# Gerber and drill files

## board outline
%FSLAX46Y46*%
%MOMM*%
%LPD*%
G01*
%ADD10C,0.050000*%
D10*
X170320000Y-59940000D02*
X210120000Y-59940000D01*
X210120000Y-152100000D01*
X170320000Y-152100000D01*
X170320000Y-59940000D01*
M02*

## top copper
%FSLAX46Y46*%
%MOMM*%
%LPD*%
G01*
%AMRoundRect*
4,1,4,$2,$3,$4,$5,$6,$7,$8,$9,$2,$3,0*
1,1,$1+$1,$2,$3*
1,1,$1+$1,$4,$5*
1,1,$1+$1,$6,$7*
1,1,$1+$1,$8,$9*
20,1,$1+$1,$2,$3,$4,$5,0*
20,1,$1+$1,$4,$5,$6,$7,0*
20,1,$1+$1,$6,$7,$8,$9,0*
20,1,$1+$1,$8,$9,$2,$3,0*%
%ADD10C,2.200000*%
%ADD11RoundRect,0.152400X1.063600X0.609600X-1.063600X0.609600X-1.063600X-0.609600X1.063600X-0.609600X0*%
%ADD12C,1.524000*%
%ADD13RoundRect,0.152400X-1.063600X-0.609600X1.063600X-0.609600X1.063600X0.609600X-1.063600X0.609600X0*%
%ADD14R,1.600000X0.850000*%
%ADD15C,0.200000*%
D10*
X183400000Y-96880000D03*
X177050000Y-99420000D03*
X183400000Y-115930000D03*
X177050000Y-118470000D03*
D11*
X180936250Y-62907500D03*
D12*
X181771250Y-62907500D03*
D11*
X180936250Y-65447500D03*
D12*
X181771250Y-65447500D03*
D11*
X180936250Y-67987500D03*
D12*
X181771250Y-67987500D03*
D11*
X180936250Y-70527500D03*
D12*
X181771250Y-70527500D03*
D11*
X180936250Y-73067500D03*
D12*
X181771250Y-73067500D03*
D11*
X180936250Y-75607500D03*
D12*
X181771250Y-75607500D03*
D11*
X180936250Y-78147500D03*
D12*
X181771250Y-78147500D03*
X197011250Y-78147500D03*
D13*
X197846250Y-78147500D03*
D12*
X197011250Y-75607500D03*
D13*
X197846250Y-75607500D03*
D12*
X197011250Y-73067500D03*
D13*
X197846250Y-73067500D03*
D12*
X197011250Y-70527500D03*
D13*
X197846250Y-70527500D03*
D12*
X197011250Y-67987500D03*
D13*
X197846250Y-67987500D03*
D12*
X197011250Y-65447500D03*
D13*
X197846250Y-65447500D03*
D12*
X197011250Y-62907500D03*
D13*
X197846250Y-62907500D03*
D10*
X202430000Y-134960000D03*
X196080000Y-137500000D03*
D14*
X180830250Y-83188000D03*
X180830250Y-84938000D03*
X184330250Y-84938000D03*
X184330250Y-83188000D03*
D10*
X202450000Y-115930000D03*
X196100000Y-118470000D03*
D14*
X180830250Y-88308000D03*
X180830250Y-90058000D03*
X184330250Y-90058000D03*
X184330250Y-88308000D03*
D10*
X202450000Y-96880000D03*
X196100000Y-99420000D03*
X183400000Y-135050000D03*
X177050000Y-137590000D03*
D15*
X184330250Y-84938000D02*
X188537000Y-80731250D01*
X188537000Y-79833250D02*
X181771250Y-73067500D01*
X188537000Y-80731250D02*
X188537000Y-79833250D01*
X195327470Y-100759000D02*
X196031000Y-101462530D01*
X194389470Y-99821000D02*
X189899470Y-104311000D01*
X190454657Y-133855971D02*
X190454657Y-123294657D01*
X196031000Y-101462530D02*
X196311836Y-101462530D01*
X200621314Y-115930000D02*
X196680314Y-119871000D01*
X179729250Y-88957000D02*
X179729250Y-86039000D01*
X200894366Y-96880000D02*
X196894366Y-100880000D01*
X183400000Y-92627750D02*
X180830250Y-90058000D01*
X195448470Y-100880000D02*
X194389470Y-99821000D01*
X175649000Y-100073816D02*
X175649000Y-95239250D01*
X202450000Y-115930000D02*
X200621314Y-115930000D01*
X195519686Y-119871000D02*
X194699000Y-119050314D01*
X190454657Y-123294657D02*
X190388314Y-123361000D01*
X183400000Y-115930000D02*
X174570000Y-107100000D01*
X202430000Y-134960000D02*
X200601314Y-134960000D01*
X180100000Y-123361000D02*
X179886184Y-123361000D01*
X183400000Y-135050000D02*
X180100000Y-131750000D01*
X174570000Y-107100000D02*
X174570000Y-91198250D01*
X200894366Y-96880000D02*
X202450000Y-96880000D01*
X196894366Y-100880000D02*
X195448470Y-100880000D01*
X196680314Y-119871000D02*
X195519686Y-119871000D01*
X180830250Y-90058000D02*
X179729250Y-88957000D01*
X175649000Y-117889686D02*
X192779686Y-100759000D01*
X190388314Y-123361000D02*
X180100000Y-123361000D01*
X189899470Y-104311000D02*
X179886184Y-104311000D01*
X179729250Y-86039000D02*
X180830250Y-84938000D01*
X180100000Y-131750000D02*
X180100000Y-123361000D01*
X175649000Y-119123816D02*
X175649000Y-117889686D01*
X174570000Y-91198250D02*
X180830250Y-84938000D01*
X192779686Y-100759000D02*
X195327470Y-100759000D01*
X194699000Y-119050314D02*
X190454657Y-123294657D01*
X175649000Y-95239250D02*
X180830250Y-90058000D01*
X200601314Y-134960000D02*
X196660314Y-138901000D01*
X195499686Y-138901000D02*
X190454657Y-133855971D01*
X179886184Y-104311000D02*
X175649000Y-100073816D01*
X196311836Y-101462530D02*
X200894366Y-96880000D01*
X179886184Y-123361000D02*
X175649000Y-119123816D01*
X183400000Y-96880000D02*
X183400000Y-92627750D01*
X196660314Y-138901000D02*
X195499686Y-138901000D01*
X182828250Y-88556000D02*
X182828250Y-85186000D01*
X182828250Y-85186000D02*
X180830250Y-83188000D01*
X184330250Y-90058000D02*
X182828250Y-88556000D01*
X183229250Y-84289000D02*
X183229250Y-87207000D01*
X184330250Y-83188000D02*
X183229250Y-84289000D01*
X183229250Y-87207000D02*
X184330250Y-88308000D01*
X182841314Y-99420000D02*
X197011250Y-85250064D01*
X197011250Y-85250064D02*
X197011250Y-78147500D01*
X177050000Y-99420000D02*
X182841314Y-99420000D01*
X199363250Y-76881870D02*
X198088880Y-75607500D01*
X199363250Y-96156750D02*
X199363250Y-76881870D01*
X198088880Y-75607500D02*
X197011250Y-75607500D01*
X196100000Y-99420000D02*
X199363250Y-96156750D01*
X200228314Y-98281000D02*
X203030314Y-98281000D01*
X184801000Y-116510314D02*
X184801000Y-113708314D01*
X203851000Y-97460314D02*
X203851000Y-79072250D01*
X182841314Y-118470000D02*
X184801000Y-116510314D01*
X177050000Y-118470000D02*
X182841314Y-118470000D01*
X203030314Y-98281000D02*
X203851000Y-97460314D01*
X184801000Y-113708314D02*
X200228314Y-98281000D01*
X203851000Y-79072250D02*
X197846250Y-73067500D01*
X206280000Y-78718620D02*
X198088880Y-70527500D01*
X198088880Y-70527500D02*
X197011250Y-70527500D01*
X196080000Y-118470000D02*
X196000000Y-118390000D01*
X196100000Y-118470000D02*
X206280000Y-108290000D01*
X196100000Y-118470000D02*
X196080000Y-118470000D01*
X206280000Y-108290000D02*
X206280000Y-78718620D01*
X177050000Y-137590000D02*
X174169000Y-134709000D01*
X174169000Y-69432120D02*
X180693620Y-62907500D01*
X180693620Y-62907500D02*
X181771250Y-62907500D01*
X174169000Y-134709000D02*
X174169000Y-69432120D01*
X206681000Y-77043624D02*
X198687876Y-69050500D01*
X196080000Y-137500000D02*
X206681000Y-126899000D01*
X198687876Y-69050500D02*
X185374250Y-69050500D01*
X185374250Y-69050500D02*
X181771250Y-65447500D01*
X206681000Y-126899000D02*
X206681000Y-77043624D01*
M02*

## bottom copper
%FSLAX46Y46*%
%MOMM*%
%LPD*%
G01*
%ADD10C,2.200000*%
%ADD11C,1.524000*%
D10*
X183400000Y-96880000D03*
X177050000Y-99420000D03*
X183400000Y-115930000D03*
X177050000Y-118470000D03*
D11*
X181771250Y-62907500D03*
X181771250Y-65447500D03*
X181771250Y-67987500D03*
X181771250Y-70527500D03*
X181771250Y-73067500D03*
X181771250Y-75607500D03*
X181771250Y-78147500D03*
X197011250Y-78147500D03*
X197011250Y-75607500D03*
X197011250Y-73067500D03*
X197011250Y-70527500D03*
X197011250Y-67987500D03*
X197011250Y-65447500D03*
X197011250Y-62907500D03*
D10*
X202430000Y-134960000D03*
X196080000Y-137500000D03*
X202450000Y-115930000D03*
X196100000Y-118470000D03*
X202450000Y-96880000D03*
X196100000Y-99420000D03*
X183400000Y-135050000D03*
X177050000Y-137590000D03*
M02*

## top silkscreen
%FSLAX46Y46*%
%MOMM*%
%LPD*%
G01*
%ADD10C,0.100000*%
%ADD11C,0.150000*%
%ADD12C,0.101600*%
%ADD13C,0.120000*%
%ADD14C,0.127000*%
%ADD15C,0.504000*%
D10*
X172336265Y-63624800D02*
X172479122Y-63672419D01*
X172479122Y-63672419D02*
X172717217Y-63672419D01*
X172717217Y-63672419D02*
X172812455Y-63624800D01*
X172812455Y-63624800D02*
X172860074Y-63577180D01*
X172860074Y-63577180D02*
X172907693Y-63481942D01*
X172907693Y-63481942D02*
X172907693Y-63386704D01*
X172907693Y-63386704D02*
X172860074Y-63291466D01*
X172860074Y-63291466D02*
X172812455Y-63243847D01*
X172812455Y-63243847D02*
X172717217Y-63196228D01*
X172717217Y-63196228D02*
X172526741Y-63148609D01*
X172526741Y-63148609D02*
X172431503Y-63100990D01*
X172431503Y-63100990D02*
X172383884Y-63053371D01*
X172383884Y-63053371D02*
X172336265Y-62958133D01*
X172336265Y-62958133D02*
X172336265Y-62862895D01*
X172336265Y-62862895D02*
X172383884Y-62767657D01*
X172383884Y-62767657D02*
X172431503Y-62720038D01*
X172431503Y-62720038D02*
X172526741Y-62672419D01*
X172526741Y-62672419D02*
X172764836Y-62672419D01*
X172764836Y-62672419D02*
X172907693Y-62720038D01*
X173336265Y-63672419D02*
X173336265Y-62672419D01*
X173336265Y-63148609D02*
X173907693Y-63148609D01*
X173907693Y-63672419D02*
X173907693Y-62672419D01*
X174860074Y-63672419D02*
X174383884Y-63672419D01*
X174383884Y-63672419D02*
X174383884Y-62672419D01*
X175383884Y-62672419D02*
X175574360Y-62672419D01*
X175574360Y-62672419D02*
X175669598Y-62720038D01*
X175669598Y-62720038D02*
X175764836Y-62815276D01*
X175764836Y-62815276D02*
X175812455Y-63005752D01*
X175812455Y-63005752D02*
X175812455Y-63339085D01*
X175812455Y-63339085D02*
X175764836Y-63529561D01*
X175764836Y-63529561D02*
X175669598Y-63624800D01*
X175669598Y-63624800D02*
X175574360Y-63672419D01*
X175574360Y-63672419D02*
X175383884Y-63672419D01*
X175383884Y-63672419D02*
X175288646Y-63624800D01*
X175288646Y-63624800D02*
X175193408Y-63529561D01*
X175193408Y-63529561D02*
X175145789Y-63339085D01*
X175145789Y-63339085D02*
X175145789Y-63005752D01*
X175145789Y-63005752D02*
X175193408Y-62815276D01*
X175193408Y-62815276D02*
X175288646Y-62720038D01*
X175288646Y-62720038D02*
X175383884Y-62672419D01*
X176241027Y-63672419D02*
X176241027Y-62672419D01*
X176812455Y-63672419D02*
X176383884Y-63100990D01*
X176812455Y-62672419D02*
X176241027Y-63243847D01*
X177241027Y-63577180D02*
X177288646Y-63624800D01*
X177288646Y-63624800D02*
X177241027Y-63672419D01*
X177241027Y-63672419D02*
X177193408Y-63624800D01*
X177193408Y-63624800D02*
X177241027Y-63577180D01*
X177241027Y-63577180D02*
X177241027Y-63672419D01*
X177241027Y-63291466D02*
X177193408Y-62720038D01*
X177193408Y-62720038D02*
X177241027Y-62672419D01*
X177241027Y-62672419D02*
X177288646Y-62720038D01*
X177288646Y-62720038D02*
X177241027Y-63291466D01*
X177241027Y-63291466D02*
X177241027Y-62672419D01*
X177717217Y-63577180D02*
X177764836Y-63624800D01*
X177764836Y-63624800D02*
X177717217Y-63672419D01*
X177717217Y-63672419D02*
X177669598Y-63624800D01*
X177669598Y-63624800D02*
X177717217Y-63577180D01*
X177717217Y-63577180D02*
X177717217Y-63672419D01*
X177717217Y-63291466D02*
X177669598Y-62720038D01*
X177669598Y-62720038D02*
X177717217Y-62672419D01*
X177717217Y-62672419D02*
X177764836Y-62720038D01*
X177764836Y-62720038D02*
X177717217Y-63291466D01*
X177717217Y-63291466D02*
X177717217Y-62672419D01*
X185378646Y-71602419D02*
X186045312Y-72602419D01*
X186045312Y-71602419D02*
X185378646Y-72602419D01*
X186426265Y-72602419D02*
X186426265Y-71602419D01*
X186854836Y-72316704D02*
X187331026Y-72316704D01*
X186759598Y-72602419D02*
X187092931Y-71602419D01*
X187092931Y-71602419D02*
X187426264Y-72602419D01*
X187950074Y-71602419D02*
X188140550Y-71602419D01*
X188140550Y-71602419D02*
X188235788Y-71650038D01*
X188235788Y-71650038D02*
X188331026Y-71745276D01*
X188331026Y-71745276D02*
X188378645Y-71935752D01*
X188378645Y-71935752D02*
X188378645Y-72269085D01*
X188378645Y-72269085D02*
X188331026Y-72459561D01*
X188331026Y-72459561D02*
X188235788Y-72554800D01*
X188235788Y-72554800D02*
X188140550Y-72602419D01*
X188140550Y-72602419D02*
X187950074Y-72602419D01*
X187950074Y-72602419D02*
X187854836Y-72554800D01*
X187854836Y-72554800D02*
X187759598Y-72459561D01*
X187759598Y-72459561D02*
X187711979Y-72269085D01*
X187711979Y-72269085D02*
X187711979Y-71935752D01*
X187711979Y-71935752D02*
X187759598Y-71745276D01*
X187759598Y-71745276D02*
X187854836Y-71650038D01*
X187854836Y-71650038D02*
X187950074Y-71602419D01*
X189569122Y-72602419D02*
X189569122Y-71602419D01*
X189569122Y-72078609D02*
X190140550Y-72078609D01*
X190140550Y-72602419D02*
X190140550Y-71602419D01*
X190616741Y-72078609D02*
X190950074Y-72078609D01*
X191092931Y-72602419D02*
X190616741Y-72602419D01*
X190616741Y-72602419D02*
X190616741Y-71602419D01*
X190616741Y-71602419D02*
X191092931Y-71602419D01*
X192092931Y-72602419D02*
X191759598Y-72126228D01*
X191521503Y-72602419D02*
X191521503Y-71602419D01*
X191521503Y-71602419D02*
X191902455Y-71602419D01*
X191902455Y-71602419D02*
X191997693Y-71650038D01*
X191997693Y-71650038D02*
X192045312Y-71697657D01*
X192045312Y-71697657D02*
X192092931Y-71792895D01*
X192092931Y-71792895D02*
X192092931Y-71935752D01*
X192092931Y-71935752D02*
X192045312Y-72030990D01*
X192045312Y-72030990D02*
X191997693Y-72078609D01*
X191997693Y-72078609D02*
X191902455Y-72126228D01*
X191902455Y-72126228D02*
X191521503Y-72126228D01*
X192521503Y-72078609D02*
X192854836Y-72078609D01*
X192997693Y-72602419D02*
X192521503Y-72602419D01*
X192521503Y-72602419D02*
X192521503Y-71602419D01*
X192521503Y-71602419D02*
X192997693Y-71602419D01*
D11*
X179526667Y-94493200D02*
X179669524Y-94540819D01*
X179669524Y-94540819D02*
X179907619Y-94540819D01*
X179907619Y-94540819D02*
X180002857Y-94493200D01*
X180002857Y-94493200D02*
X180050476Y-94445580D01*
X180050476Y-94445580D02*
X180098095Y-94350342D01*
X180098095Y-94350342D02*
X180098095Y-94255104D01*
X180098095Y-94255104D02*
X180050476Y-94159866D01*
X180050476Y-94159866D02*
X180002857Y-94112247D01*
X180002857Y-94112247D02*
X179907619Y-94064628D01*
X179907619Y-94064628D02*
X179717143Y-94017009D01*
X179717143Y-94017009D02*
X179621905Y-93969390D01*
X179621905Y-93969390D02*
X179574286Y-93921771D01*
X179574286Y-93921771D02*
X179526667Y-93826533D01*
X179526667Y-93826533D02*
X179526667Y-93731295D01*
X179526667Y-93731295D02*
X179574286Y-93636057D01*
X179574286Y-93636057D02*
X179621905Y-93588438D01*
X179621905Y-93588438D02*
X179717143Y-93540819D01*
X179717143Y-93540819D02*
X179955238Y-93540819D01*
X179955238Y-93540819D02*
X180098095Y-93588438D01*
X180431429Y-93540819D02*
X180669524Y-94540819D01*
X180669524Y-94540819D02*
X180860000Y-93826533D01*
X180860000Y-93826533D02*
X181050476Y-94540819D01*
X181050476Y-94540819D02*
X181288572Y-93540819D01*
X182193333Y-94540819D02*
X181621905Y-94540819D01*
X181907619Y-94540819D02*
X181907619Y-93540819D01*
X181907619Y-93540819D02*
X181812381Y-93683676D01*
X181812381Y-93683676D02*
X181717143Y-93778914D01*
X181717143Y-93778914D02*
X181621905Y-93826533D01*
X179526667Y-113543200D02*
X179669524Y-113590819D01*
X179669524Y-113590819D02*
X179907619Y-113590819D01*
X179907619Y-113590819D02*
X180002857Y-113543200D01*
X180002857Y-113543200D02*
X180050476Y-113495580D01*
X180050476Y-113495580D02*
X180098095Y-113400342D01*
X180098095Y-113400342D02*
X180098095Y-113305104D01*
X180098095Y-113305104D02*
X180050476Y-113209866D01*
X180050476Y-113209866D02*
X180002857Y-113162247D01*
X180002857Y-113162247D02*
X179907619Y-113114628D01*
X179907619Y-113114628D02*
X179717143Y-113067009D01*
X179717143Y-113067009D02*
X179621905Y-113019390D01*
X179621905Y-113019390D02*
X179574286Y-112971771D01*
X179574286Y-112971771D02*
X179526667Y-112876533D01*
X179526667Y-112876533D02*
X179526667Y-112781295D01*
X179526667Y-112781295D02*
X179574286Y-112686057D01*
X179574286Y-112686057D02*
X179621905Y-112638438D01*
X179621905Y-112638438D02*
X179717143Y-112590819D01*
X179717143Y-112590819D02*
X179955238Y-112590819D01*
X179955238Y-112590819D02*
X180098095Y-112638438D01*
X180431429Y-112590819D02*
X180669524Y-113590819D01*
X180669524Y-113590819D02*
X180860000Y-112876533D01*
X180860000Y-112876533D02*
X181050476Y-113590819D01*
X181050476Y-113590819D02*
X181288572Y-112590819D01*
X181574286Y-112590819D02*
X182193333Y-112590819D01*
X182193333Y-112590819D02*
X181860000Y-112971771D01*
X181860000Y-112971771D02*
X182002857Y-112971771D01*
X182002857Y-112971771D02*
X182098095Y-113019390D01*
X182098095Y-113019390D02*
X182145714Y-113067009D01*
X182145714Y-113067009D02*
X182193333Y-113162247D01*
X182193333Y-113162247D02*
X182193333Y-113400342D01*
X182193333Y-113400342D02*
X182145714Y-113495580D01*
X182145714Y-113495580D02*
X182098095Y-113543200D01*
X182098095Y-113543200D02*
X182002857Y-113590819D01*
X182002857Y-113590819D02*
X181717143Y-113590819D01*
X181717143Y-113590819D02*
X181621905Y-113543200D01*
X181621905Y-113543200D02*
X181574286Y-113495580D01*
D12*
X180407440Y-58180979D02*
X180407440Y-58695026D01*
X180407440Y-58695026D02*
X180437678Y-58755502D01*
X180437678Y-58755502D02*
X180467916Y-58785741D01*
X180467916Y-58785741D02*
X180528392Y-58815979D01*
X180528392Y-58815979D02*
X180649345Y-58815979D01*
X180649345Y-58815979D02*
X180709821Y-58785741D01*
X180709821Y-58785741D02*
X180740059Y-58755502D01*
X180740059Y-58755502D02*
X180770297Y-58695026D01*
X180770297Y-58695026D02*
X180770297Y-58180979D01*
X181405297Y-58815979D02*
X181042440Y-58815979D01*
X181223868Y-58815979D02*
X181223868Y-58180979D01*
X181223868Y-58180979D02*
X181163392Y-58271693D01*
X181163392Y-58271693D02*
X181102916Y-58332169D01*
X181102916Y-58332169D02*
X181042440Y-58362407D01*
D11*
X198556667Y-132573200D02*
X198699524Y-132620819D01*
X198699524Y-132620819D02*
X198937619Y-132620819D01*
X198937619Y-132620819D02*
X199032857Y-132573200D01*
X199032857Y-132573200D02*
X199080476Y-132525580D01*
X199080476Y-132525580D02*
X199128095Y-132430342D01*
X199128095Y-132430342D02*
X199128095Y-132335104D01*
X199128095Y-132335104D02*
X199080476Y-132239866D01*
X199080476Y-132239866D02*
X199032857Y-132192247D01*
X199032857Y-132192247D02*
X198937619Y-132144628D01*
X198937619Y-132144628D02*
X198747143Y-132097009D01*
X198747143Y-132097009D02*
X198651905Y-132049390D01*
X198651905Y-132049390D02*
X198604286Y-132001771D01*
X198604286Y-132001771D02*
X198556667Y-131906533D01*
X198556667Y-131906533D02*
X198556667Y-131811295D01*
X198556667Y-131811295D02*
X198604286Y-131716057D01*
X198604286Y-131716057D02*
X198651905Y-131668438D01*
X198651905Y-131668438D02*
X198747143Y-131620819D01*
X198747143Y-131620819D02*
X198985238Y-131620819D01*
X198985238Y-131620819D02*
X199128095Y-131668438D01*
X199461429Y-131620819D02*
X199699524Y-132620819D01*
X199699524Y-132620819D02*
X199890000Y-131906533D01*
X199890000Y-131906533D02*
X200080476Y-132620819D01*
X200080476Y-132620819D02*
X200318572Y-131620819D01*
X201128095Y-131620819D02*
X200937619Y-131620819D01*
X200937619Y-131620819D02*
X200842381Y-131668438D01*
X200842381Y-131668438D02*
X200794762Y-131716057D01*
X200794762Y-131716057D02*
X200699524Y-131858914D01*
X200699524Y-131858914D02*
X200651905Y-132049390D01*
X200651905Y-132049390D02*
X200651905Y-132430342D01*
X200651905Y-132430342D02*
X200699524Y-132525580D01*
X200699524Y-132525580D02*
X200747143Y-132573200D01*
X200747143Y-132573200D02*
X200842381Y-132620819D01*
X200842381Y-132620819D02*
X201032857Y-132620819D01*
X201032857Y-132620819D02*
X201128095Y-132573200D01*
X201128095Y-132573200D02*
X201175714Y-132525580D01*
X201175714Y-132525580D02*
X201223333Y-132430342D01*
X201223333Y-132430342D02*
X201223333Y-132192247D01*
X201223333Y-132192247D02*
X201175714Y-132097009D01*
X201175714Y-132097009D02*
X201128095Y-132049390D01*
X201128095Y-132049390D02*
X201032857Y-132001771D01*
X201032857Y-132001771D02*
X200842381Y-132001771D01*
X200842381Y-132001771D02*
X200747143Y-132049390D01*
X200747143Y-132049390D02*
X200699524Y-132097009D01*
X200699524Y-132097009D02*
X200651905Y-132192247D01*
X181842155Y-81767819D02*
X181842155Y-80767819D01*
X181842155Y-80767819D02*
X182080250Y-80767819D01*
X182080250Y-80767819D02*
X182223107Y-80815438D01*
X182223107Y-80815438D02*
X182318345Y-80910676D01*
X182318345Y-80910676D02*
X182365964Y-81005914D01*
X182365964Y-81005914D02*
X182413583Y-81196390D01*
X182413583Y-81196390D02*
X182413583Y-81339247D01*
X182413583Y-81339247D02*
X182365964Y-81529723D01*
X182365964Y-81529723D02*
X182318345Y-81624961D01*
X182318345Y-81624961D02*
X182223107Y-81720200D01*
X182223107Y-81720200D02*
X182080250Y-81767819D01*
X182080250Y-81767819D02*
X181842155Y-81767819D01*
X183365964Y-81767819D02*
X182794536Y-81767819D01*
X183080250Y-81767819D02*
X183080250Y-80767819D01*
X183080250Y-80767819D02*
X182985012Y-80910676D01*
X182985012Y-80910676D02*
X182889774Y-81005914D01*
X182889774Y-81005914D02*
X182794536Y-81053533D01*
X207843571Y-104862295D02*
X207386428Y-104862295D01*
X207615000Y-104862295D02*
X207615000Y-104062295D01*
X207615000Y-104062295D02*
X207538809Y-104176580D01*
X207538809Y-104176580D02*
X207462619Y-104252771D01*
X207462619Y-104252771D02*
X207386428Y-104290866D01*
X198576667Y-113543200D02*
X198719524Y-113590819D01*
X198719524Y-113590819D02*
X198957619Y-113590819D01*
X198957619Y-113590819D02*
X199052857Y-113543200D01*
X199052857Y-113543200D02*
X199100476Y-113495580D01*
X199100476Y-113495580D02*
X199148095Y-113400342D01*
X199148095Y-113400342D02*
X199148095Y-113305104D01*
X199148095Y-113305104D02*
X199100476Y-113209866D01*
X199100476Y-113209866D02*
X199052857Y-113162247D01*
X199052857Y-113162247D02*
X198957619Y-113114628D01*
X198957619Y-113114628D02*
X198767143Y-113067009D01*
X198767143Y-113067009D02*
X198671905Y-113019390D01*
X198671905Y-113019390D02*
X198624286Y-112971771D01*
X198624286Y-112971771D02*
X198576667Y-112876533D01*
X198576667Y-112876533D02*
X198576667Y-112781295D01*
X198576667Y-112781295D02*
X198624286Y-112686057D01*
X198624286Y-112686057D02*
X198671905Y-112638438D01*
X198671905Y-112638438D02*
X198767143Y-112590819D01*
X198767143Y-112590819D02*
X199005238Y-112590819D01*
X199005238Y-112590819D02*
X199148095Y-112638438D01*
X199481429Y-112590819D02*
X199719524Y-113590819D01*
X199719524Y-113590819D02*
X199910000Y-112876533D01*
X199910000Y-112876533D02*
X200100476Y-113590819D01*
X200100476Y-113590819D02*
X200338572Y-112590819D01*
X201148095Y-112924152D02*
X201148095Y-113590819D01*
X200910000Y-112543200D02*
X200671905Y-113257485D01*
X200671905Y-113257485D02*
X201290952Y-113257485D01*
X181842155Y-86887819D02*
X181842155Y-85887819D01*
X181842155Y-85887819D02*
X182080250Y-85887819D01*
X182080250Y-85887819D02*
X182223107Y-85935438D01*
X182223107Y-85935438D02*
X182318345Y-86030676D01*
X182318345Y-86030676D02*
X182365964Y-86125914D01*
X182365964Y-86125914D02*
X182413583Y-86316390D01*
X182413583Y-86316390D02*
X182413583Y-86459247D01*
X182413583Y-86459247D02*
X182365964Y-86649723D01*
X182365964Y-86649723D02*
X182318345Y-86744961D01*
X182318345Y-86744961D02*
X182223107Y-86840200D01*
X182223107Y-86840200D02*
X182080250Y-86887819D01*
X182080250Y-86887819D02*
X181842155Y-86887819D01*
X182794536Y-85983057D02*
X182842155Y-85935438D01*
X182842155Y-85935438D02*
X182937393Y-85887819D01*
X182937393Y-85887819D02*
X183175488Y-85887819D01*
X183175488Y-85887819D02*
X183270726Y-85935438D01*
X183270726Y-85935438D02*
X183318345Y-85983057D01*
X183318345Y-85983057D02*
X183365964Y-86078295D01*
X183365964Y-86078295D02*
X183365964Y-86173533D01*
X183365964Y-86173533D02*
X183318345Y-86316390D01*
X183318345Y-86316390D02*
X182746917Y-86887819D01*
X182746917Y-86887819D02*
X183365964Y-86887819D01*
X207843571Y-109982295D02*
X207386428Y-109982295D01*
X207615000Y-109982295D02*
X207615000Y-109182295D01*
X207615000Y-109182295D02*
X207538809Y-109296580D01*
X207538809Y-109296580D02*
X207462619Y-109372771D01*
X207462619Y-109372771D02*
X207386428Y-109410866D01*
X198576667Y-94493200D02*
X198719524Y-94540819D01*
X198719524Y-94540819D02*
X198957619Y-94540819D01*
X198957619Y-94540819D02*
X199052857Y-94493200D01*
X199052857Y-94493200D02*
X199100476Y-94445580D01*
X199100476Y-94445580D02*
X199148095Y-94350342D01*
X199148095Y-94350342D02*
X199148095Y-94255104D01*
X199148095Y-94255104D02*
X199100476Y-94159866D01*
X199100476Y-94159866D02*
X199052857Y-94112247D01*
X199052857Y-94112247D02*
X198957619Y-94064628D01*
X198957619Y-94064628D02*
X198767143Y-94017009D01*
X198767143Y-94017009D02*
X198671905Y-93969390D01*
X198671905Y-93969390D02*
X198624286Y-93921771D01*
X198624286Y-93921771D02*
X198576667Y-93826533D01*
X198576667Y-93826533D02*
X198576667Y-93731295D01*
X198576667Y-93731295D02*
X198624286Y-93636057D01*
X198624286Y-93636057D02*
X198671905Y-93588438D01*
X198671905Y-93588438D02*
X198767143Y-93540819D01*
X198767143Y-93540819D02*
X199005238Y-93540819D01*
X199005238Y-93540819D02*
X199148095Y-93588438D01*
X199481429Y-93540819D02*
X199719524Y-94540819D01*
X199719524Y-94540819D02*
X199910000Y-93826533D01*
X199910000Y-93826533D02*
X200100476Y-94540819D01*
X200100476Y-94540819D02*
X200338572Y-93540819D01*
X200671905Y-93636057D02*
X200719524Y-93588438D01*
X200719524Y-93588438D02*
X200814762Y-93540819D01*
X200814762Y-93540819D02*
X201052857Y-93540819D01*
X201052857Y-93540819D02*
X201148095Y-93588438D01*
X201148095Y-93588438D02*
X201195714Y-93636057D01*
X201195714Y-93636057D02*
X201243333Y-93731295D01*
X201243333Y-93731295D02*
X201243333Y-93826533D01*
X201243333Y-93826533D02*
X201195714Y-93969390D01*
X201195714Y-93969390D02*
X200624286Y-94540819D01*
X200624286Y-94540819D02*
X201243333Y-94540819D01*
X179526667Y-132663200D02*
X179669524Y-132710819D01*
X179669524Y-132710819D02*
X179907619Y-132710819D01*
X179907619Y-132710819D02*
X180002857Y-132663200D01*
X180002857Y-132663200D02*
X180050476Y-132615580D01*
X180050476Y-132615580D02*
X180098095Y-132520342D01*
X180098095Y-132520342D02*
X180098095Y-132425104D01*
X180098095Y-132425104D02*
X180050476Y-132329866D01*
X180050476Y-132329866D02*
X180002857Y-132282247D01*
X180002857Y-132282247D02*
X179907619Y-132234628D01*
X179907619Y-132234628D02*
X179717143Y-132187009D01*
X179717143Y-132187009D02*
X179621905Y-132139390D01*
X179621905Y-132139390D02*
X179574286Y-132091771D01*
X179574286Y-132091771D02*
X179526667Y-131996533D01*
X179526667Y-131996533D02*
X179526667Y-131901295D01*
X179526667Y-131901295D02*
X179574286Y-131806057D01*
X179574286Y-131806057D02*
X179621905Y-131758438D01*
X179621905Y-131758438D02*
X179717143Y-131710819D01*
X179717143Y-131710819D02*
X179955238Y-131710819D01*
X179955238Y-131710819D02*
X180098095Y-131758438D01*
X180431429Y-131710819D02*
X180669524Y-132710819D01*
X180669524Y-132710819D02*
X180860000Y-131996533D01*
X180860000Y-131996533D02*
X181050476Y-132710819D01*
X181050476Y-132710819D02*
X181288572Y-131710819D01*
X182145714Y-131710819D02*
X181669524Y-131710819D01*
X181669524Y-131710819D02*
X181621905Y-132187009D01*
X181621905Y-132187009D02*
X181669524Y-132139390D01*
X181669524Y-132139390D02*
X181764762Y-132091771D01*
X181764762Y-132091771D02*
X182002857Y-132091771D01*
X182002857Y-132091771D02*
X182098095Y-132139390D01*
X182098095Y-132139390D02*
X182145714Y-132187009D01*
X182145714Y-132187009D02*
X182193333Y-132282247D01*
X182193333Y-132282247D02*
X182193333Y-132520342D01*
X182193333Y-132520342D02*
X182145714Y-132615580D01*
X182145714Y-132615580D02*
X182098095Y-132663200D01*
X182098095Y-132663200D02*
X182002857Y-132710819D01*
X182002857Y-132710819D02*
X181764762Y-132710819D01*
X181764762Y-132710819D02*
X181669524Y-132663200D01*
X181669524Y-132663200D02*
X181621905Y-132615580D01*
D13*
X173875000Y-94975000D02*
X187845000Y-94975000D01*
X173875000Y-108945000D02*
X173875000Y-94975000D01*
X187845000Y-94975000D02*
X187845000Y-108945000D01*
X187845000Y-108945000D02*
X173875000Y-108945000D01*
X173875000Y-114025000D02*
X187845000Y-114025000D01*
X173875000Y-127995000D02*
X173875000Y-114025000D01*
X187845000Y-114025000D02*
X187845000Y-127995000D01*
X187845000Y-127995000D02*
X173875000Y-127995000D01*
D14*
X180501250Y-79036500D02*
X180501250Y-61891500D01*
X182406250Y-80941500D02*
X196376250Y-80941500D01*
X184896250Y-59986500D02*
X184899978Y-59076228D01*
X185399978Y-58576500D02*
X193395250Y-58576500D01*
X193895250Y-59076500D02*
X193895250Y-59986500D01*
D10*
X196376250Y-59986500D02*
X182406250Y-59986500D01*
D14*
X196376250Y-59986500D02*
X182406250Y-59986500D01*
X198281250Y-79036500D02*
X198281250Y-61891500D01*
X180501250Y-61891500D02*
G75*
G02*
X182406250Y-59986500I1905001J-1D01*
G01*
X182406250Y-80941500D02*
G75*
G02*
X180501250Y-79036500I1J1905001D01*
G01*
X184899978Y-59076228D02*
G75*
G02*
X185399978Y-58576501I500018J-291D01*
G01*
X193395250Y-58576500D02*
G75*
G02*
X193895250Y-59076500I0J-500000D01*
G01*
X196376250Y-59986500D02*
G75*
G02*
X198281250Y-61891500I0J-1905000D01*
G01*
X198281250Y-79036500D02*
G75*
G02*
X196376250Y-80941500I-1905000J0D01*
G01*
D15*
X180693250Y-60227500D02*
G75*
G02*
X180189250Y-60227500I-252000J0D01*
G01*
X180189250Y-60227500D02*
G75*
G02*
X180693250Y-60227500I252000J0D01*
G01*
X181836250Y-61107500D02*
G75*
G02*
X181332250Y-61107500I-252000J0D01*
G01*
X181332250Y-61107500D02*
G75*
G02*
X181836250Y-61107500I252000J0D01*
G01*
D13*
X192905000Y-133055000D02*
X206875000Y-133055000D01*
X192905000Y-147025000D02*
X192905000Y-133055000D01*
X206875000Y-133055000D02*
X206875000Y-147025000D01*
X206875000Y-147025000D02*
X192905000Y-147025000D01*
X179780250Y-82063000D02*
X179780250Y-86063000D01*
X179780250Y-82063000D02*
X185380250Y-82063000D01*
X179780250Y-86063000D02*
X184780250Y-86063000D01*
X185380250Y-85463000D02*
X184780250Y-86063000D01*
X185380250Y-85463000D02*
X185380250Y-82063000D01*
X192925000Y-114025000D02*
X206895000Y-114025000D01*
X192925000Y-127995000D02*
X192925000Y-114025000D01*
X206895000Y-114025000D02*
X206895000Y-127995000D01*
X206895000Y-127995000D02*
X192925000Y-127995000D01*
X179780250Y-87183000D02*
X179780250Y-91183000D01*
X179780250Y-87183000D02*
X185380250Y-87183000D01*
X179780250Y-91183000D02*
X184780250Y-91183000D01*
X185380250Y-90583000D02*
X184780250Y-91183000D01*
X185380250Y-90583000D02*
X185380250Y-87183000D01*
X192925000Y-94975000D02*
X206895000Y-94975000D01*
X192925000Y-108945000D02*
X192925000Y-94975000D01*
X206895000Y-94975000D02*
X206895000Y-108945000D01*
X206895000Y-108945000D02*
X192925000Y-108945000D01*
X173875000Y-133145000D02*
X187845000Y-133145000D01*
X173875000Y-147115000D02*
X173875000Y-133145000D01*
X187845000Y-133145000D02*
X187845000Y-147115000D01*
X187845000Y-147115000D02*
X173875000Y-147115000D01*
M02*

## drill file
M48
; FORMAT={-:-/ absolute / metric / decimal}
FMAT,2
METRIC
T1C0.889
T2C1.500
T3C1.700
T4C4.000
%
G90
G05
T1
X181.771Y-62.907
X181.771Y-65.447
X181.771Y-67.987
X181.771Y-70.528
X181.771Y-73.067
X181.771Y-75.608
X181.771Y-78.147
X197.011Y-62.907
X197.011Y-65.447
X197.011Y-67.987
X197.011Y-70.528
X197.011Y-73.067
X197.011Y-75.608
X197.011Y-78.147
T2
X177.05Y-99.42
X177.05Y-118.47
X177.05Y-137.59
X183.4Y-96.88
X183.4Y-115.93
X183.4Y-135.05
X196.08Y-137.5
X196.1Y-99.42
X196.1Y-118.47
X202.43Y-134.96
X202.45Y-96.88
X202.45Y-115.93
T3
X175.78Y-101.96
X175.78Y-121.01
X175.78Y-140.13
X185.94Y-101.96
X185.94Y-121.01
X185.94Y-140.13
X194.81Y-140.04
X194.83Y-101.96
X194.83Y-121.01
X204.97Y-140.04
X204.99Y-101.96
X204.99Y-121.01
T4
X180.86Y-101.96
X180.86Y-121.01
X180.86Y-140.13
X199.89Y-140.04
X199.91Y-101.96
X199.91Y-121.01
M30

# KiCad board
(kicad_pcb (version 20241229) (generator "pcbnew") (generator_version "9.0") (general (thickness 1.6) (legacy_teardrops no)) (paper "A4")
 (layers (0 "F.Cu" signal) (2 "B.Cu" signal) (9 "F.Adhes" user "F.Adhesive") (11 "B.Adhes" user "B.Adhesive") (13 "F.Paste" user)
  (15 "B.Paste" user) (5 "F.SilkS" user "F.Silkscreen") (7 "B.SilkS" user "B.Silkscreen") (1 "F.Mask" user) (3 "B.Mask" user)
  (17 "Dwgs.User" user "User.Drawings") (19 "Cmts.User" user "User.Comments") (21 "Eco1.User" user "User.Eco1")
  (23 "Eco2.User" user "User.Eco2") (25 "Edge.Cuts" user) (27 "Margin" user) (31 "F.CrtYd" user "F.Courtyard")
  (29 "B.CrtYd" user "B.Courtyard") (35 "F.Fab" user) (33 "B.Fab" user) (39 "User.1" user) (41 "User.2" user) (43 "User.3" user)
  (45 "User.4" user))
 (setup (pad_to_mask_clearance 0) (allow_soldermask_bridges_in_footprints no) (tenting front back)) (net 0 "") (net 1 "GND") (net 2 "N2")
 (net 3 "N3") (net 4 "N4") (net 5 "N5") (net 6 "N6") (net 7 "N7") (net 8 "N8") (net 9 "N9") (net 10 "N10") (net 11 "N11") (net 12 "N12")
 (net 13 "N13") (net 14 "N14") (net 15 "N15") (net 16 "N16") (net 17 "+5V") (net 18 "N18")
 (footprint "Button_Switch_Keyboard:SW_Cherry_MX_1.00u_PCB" (layer "F.Cu") (at 183.4 96.88)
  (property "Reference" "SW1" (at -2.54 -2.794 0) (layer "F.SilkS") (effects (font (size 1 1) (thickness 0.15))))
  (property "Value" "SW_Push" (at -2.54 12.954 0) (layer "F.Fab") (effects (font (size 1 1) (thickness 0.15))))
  (fp_line (start -9.525 -1.905) (end 4.445 -1.905) (stroke (width 0.12) (type solid)) (layer "F.SilkS"))
  (fp_line (start -9.525 12.065) (end -9.525 -1.905) (stroke (width 0.12) (type solid)) (layer "F.SilkS"))
  (fp_line (start 4.445 -1.905) (end 4.445 12.065) (stroke (width 0.12) (type solid)) (layer "F.SilkS"))
  (fp_line (start 4.445 12.065) (end -9.525 12.065) (stroke (width 0.12) (type solid)) (layer "F.SilkS"))
  (pad "" np_thru_hole circle (at -7.62 5.08) (size 1.7 1.7) (drill 1.7) (layers "*.Cu" "*.Mask"))
  (pad "" np_thru_hole circle (at -2.54 5.08) (size 4 4) (drill 4) (layers "*.Cu" "*.Mask"))
  (pad "" np_thru_hole circle (at 2.54 5.08) (size 1.7 1.7) (drill 1.7) (layers "*.Cu" "*.Mask"))
  (pad "1" thru_hole circle (at 0 0) (size 2.2 2.2) (drill 1.5) (layers "*.Cu" "*.Mask") (remove_unused_layers no) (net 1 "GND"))
  (pad "2" thru_hole circle (at -6.35 2.54) (size 2.2 2.2) (drill 1.5) (layers "*.Cu" "*.Mask") (remove_unused_layers no) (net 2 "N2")))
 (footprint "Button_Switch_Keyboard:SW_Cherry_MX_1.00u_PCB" (layer "F.Cu") (at 183.4 115.93)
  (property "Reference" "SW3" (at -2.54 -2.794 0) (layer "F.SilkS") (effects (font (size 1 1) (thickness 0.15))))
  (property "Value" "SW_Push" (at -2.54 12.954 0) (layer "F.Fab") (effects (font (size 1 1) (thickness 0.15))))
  (fp_line (start -9.525 -1.905) (end 4.445 -1.905) (stroke (width 0.12) (type solid)) (layer "F.SilkS"))
  (fp_line (start -9.525 12.065) (end -9.525 -1.905) (stroke (width 0.12) (type solid)) (layer "F.SilkS"))
  (fp_line (start 4.445 -1.905) (end 4.445 12.065) (stroke (width 0.12) (type solid)) (layer "F.SilkS"))
  (fp_line (start 4.445 12.065) (end -9.525 12.065) (stroke (width 0.12) (type solid)) (layer "F.SilkS"))
  (pad "" np_thru_hole circle (at -7.62 5.08) (size 1.7 1.7) (drill 1.7) (layers "*.Cu" "*.Mask"))
  (pad "" np_thru_hole circle (at -2.54 5.08) (size 4 4) (drill 4) (layers "*.Cu" "*.Mask"))
  (pad "" np_thru_hole circle (at 2.54 5.08) (size 1.7 1.7) (drill 1.7) (layers "*.Cu" "*.Mask"))
  (pad "1" thru_hole circle (at 0 0) (size 2.2 2.2) (drill 1.5) (layers "*.Cu" "*.Mask") (remove_unused_layers no) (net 1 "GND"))
  (pad "2" thru_hole circle (at -6.35 2.54) (size 2.2 2.2) (drill 1.5) (layers "*.Cu" "*.Mask") (remove_unused_layers no) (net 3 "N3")))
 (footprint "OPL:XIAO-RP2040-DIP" (layer "F.Cu") (at 189.39125 70.5275)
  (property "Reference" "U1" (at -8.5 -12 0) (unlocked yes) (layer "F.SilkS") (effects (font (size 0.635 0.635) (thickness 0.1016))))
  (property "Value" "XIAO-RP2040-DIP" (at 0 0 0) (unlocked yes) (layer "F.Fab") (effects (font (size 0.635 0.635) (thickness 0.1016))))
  (fp_line (start -8.89 8.509) (end -8.89 -8.636) (stroke (width 0.127) (type solid)) (layer "F.SilkS"))
  (fp_line (start -6.985 10.414) (end 6.985 10.414) (stroke (width 0.127) (type solid)) (layer "F.SilkS"))
  (fp_line (start -4.495 -10.541) (end -4.491272 -11.451272) (stroke (width 0.127) (type solid)) (layer "F.SilkS"))
  (fp_line (start -3.991272 -11.951) (end 4.004 -11.951) (stroke (width 0.127) (type solid)) (layer "F.SilkS"))
  (fp_line (start 4.504 -11.451) (end 4.504 -10.541) (stroke (width 0.127) (type solid)) (layer "F.SilkS"))
  (fp_line (start 6.985 -10.541) (end -6.985 -10.541) (stroke (width 0.1) (type solid)) (layer "F.SilkS"))
  (fp_line (start 6.985 -10.541) (end -6.985 -10.541) (stroke (width 0.127) (type solid)) (layer "F.SilkS"))
  (fp_line (start 8.89 8.509) (end 8.89 -8.636) (stroke (width 0.127) (type solid)) (layer "F.SilkS"))
  (fp_arc (start -8.89 -8.636) (mid -8.332038 -9.983038) (end -6.985 -10.541) (stroke (width 0.127) (type solid)) (layer "F.SilkS"))
  (fp_arc (start -6.985 10.414) (mid -8.332038 9.856038) (end -8.89 8.509) (stroke (width 0.127) (type solid)) (layer "F.SilkS"))
  (fp_arc (start -4.491272 -11.451272) (mid -4.344728 -11.80464) (end -3.991272 -11.951) (stroke (width 0.127) (type default))
   (layer "F.SilkS"))
  (fp_arc (start 4.004 -11.951) (mid 4.357553 -11.804553) (end 4.504 -11.451) (stroke (width 0.127) (type default)) (layer "F.SilkS"))
  (fp_arc (start 6.985 -10.541) (mid 8.332038 -9.983038) (end 8.89 -8.636) (stroke (width 0.127) (type solid)) (layer "F.SilkS"))
  (fp_arc (start 8.89 8.509) (mid 8.332038 9.856038) (end 6.985 10.414) (stroke (width 0.127) (type solid)) (layer "F.SilkS"))
  (fp_circle (center -8.95 -10.3) (end -8.95 -10.554) (stroke (width 0.5) (type solid)) (fill yes) (layer "F.SilkS"))
  (fp_circle (center -7.807 -9.42) (end -7.807 -9.674) (stroke (width 0.5) (type solid)) (fill yes) (layer "F.SilkS"))
  (pad "1" smd roundrect (at -8.455 -7.62 180) (size 2.432 1.524) (layers "F.Cu" "F.Mask") (roundrect_rratio 0.1) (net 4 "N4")
   (thermal_bridge_angle 45))
  (pad "1" thru_hole circle (at -7.62 -7.62 180) (size 1.524 1.524) (drill 0.889) (layers "*.Cu" "*.Mask") (remove_unused_layers no)
   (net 4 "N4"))
  (pad "2" smd roundrect (at -8.455 -5.08 180) (size 2.432 1.524) (layers "F.Cu" "F.Mask") (roundrect_rratio 0.1) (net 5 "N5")
   (thermal_bridge_angle 45))
  (pad "2" thru_hole circle (at -7.62 -5.08 180) (size 1.524 1.524) (drill 0.889) (layers "*.Cu" "*.Mask") (remove_unused_layers no)
   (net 5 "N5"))
  (pad "3" smd roundrect (at -8.455 -2.54 180) (size 2.432 1.524) (layers "F.Cu" "F.Mask") (roundrect_rratio 0.1) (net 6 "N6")
   (thermal_bridge_angle 45))
  (pad "3" thru_hole circle (at -7.62 -2.54 180) (size 1.524 1.524) (drill 0.889) (layers "*.Cu" "*.Mask") (remove_unused_layers no)
   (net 6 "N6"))
  (pad "4" smd roundrect (at -8.455 0 180) (size 2.432 1.524) (layers "F.Cu" "F.Mask") (roundrect_rratio 0.1) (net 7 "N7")
   (thermal_bridge_angle 45))
  (pad "4" thru_hole circle (at -7.62 0 180) (size 1.524 1.524) (drill 0.889) (layers "*.Cu" "*.Mask") (remove_unused_layers no)
   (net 7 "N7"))
  (pad "5" smd roundrect (at -8.455 2.54 180) (size 2.432 1.524) (layers "F.Cu" "F.Mask") (roundrect_rratio 0.1) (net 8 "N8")
   (thermal_bridge_angle 45))
  (pad "5" thru_hole circle (at -7.62 2.54 180) (size 1.524 1.524) (drill 0.889) (layers "*.Cu" "*.Mask") (remove_unused_layers no)
   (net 8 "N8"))
  (pad "6" smd roundrect (at -8.455 5.08 180) (size 2.432 1.524) (layers "F.Cu" "F.Mask") (roundrect_rratio 0.1) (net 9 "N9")
   (thermal_bridge_angle 45))
  (pad "6" thru_hole circle (at -7.62 5.08 180) (size 1.524 1.524) (drill 0.889) (layers "*.Cu" "*.Mask") (remove_unused_layers no)
   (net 9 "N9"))
  (pad "7" smd roundrect (at -8.455 7.62 180) (size 2.432 1.524) (layers "F.Cu" "F.Mask") (roundrect_rratio 0.1) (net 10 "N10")
   (thermal_bridge_angle 45))
  (pad "7" thru_hole circle (at -7.62 7.62 180) (size 1.524 1.524) (drill 0.889) (layers "*.Cu" "*.Mask") (remove_unused_layers no)
   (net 10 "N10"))
  (pad "8" thru_hole circle (at 7.62 7.62) (size 1.524 1.524) (drill 0.889) (layers "*.Cu" "*.Mask") (remove_unused_layers no) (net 2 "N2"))
  (pad "8" smd roundrect (at 8.455 7.62) (size 2.432 1.524) (layers "F.Cu" "F.Mask") (roundrect_rratio 0.1) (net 2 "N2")
   (thermal_bridge_angle 45))
  (pad "9" thru_hole circle (at 7.62 5.08) (size 1.524 1.524) (drill 0.889) (layers "*.Cu" "*.Mask") (remove_unused_layers no)
   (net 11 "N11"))
  (pad "9" smd roundrect (at 8.455 5.08) (size 2.432 1.524) (layers "F.Cu" "F.Mask") (roundrect_rratio 0.1) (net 11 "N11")
   (thermal_bridge_angle 45))
  (pad "10" thru_hole circle (at 7.62 2.54) (size 1.524 1.524) (drill 0.889) (layers "*.Cu" "*.Mask") (remove_unused_layers no) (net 3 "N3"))
  (pad "10" smd roundrect (at 8.455 2.54) (size 2.432 1.524) (layers "F.Cu" "F.Mask") (roundrect_rratio 0.1) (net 3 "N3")
   (thermal_bridge_angle 45))
  (pad "11" thru_hole circle (at 7.62 0) (size 1.524 1.524) (drill 0.889) (layers "*.Cu" "*.Mask") (remove_unused_layers no) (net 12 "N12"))
  (pad "11" smd roundrect (at 8.455 0) (size 2.432 1.524) (layers "F.Cu" "F.Mask") (roundrect_rratio 0.1) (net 12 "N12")
   (thermal_bridge_angle 45))
  (pad "12" thru_hole circle (at 7.62 -2.54) (size 1.524 1.524) (drill 0.889) (layers "*.Cu" "*.Mask") (remove_unused_layers no)
   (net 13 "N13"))
  (pad "12" smd roundrect (at 8.455 -2.54) (size 2.432 1.524) (layers "F.Cu" "F.Mask") (roundrect_rratio 0.1) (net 13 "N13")
   (thermal_bridge_angle 45))
  (pad "13" thru_hole circle (at 7.62 -5.08) (size 1.524 1.524) (drill 0.889) (layers "*.Cu" "*.Mask") (remove_unused_layers no)
   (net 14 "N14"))
  (pad "13" smd roundrect (at 8.455 -5.08) (size 2.432 1.524) (layers "F.Cu" "F.Mask") (roundrect_rratio 0.1) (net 14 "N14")
   (thermal_bridge_angle 45))
  (pad "14" thru_hole circle (at 7.62 -7.62) (size 1.524 1.524) (drill 0.889) (layers "*.Cu" "*.Mask") (remove_unused_layers no)
   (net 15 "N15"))
  (pad "14" smd roundrect (at 8.455 -7.62) (size 2.432 1.524) (layers "F.Cu" "F.Mask") (roundrect_rratio 0.1) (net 15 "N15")
   (thermal_bridge_angle 45)))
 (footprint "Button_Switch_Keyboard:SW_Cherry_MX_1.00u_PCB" (layer "F.Cu") (at 202.43 134.96)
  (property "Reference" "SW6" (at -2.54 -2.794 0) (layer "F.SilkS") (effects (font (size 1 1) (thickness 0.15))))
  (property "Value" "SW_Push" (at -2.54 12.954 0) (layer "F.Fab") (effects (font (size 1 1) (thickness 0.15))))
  (fp_line (start -9.525 -1.905) (end 4.445 -1.905) (stroke (width 0.12) (type solid)) (layer "F.SilkS"))
  (fp_line (start -9.525 12.065) (end -9.525 -1.905) (stroke (width 0.12) (type solid)) (layer "F.SilkS"))
  (fp_line (start 4.445 -1.905) (end 4.445 12.065) (stroke (width 0.12) (type solid)) (layer "F.SilkS"))
  (fp_line (start 4.445 12.065) (end -9.525 12.065) (stroke (width 0.12) (type solid)) (layer "F.SilkS"))
  (pad "" np_thru_hole circle (at -7.62 5.08) (size 1.7 1.7) (drill 1.7) (layers "*.Cu" "*.Mask"))
  (pad "" np_thru_hole circle (at -2.54 5.08) (size 4 4) (drill 4) (layers "*.Cu" "*.Mask"))
  (pad "" np_thru_hole circle (at 2.54 5.08) (size 1.7 1.7) (drill 1.7) (layers "*.Cu" "*.Mask"))
  (pad "1" thru_hole circle (at 0 0) (size 2.2 2.2) (drill 1.5) (layers "*.Cu" "*.Mask") (remove_unused_layers no) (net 1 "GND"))
  (pad "2" thru_hole circle (at -6.35 2.54) (size 2.2 2.2) (drill 1.5) (layers "*.Cu" "*.Mask") (remove_unused_layers no) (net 5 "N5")))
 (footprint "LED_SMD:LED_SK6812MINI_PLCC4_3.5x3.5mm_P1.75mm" (layer "F.Cu") (at 182.58025 84.063)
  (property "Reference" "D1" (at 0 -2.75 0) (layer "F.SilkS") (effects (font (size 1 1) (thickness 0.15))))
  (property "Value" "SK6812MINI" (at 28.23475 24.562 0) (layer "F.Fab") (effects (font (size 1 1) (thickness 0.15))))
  (fp_line (start -2.8 -2) (end -2.8 2) (stroke (width 0.12) (type default)) (layer "F.SilkS"))
  (fp_line (start -2.8 -2) (end 2.8 -2) (stroke (width 0.12) (type solid)) (layer "F.SilkS"))
  (fp_line (start -2.8 2) (end 2.2 2) (stroke (width 0.12) (type solid)) (layer "F.SilkS"))
  (fp_line (start 2.8 1.4) (end 2.2 2) (stroke (width 0.12) (type default)) (layer "F.SilkS"))
  (fp_line (start 2.8 1.4) (end 2.8 -2) (stroke (width 0.12) (type solid)) (layer "F.SilkS"))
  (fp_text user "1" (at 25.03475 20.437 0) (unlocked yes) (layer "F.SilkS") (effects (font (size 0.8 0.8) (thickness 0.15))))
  (pad "1" smd rect (at -1.75 -0.875) (size 1.6 0.85) (layers "F.Cu" "F.Mask" "F.Paste") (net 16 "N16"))
  (pad "2" smd rect (at -1.75 0.875) (size 1.6 0.85) (layers "F.Cu" "F.Mask" "F.Paste") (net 1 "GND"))
  (pad "3" smd rect (at 1.75 0.875) (size 1.6 0.85) (layers "F.Cu" "F.Mask" "F.Paste") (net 8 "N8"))
  (pad "4" smd rect (at 1.75 -0.875) (size 1.6 0.85) (layers "F.Cu" "F.Mask" "F.Paste") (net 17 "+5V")))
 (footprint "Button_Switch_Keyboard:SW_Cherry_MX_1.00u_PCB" (layer "F.Cu") (at 202.45 115.93)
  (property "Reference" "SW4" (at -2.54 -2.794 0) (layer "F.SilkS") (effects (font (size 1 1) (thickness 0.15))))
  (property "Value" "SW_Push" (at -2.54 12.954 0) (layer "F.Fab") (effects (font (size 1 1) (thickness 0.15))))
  (fp_line (start -9.525 -1.905) (end 4.445 -1.905) (stroke (width 0.12) (type solid)) (layer "F.SilkS"))
  (fp_line (start -9.525 12.065) (end -9.525 -1.905) (stroke (width 0.12) (type solid)) (layer "F.SilkS"))
  (fp_line (start 4.445 -1.905) (end 4.445 12.065) (stroke (width 0.12) (type solid)) (layer "F.SilkS"))
  (fp_line (start 4.445 12.065) (end -9.525 12.065) (stroke (width 0.12) (type solid)) (layer "F.SilkS"))
  (pad "" np_thru_hole circle (at -7.62 5.08) (size 1.7 1.7) (drill 1.7) (layers "*.Cu" "*.Mask"))
  (pad "" np_thru_hole circle (at -2.54 5.08) (size 4 4) (drill 4) (layers "*.Cu" "*.Mask"))
  (pad "" np_thru_hole circle (at 2.54 5.08) (size 1.7 1.7) (drill 1.7) (layers "*.Cu" "*.Mask"))
  (pad "1" thru_hole circle (at 0 0) (size 2.2 2.2) (drill 1.5) (layers "*.Cu" "*.Mask") (remove_unused_layers no) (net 1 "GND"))
  (pad "2" thru_hole circle (at -6.35 2.54) (size 2.2 2.2) (drill 1.5) (layers "*.Cu" "*.Mask") (remove_unused_layers no) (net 12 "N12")))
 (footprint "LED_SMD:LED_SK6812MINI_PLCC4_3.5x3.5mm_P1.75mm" (layer "F.Cu") (at 182.58025 89.183)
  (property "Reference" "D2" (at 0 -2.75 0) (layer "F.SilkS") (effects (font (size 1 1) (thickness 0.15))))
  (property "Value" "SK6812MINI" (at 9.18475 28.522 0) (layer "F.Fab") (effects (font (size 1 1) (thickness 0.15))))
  (fp_line (start -2.8 -2) (end -2.8 2) (stroke (width 0.12) (type default)) (layer "F.SilkS"))
  (fp_line (start -2.8 -2) (end 2.8 -2) (stroke (width 0.12) (type solid)) (layer "F.SilkS"))
  (fp_line (start -2.8 2) (end 2.2 2) (stroke (width 0.12) (type solid)) (layer "F.SilkS"))
  (fp_line (start 2.8 1.4) (end 2.2 2) (stroke (width 0.12) (type default)) (layer "F.SilkS"))
  (fp_line (start 2.8 1.4) (end 2.8 -2) (stroke (width 0.12) (type solid)) (layer "F.SilkS"))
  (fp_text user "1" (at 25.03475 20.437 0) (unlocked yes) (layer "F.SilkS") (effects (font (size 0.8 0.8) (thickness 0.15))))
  (pad "1" smd rect (at -1.75 -0.875) (size 1.6 0.85) (layers "F.Cu" "F.Mask" "F.Paste") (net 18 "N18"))
  (pad "2" smd rect (at -1.75 0.875) (size 1.6 0.85) (layers "F.Cu" "F.Mask" "F.Paste") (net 1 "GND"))
  (pad "3" smd rect (at 1.75 0.875) (size 1.6 0.85) (layers "F.Cu" "F.Mask" "F.Paste") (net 16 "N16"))
  (pad "4" smd rect (at 1.75 -0.875) (size 1.6 0.85) (layers "F.Cu" "F.Mask" "F.Paste") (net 17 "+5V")))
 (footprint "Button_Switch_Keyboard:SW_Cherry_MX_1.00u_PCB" (layer "F.Cu") (at 202.45 96.88)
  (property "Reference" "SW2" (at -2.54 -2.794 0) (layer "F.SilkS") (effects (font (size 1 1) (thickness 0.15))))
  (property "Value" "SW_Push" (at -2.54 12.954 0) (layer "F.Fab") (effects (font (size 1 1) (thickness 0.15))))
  (fp_line (start -9.525 -1.905) (end 4.445 -1.905) (stroke (width 0.12) (type solid)) (layer "F.SilkS"))
  (fp_line (start -9.525 12.065) (end -9.525 -1.905) (stroke (width 0.12) (type solid)) (layer "F.SilkS"))
  (fp_line (start 4.445 -1.905) (end 4.445 12.065) (stroke (width 0.12) (type solid)) (layer "F.SilkS"))
  (fp_line (start 4.445 12.065) (end -9.525 12.065) (stroke (width 0.12) (type solid)) (layer "F.SilkS"))
  (pad "" np_thru_hole circle (at -7.62 5.08) (size 1.7 1.7) (drill 1.7) (layers "*.Cu" "*.Mask"))
  (pad "" np_thru_hole circle (at -2.54 5.08) (size 4 4) (drill 4) (layers "*.Cu" "*.Mask"))
  (pad "" np_thru_hole circle (at 2.54 5.08) (size 1.7 1.7) (drill 1.7) (layers "*.Cu" "*.Mask"))
  (pad "1" thru_hole circle (at 0 0) (size 2.2 2.2) (drill 1.5) (layers "*.Cu" "*.Mask") (remove_unused_layers no) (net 1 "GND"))
  (pad "2" thru_hole circle (at -6.35 2.54) (size 2.2 2.2) (drill 1.5) (layers "*.Cu" "*.Mask") (remove_unused_layers no) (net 11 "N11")))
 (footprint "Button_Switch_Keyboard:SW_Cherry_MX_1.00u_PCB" (layer "F.Cu") (at 183.4 135.05)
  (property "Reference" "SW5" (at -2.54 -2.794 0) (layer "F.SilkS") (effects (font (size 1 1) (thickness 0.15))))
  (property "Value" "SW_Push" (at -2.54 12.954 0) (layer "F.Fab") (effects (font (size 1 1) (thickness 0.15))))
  (fp_line (start -9.525 -1.905) (end 4.445 -1.905) (stroke (width 0.12) (type solid)) (layer "F.SilkS"))
  (fp_line (start -9.525 12.065) (end -9.525 -1.905) (stroke (width 0.12) (type solid)) (layer "F.SilkS"))
  (fp_line (start 4.445 -1.905) (end 4.445 12.065) (stroke (width 0.12) (type solid)) (layer "F.SilkS"))
  (fp_line (start 4.445 12.065) (end -9.525 12.065) (stroke (width 0.12) (type solid)) (layer "F.SilkS"))
  (pad "" np_thru_hole circle (at -7.62 5.08) (size 1.7 1.7) (drill 1.7) (layers "*.Cu" "*.Mask"))
  (pad "" np_thru_hole circle (at -2.54 5.08) (size 4 4) (drill 4) (layers "*.Cu" "*.Mask"))
  (pad "" np_thru_hole circle (at 2.54 5.08) (size 1.7 1.7) (drill 1.7) (layers "*.Cu" "*.Mask"))
  (pad "1" thru_hole circle (at 0 0) (size 2.2 2.2) (drill 1.5) (layers "*.Cu" "*.Mask") (remove_unused_layers no) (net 1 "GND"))
  (pad "2" thru_hole circle (at -6.35 2.54) (size 2.2 2.2) (drill 1.5) (layers "*.Cu" "*.Mask") (remove_unused_layers no) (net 4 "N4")))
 (gr_rect (start 170.32 59.94) (end 210.12 152.1) (stroke (width 0.05) (type default)) (fill no) (layer "Edge.Cuts"))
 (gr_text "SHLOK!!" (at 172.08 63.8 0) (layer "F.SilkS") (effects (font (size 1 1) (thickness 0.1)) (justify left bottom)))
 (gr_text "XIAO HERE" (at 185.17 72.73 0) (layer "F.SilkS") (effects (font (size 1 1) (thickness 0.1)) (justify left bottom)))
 (segment (start 184.33025 84.938) (end 188.537 80.73125) (width 0.2) (layer "F.Cu") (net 8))
 (segment (start 188.537 79.83325) (end 181.77125 73.0675) (width 0.2) (layer "F.Cu") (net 8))
 (segment (start 188.537 80.73125) (end 188.537 79.83325) (width 0.2) (layer "F.Cu") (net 8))
 (segment (start 195.32747 100.759) (end 196.031 101.46253) (width 0.2) (layer "F.Cu") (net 1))
 (segment (start 194.38947 99.821) (end 189.89947 104.311) (width 0.2) (layer "F.Cu") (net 1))
 (segment (start 190.454657 133.855971) (end 190.454657 123.294657) (width 0.2) (layer "F.Cu") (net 1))
 (segment (start 196.031 101.46253) (end 196.311836 101.46253) (width 0.2) (layer "F.Cu") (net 1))
 (segment (start 200.621314 115.93) (end 196.680314 119.871) (width 0.2) (layer "F.Cu") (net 1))
 (segment (start 179.72925 88.957) (end 179.72925 86.039) (width 0.2) (layer "F.Cu") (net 1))
 (segment (start 200.894366 96.88) (end 196.894366 100.88) (width 0.2) (layer "F.Cu") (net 1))
 (segment (start 183.4 92.62775) (end 180.83025 90.058) (width 0.2) (layer "F.Cu") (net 1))
 (segment (start 195.44847 100.88) (end 194.38947 99.821) (width 0.2) (layer "F.Cu") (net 1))
 (segment (start 175.649 100.073816) (end 175.649 95.23925) (width 0.2) (layer "F.Cu") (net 1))
 (segment (start 202.45 115.93) (end 200.621314 115.93) (width 0.2) (layer "F.Cu") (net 1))
 (segment (start 195.519686 119.871) (end 194.699 119.050314) (width 0.2) (layer "F.Cu") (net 1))
 (segment (start 190.454657 123.294657) (end 190.388314 123.361) (width 0.2) (layer "F.Cu") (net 1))
 (segment (start 183.4 115.93) (end 174.57 107.1) (width 0.2) (layer "F.Cu") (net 1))
 (segment (start 202.43 134.96) (end 200.601314 134.96) (width 0.2) (layer "F.Cu") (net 1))
 (segment (start 180.1 123.361) (end 179.886184 123.361) (width 0.2) (layer "F.Cu") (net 1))
 (segment (start 183.4 135.05) (end 180.1 131.75) (width 0.2) (layer "F.Cu") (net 1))
 (segment (start 174.57 107.1) (end 174.57 91.19825) (width 0.2) (layer "F.Cu") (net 1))
 (segment (start 200.894366 96.88) (end 202.45 96.88) (width 0.2) (layer "F.Cu") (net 1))
 (segment (start 196.894366 100.88) (end 195.44847 100.88) (width 0.2) (layer "F.Cu") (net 1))
 (segment (start 196.680314 119.871) (end 195.519686 119.871) (width 0.2) (layer "F.Cu") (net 1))
 (segment (start 180.83025 90.058) (end 179.72925 88.957) (width 0.2) (layer "F.Cu") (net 1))
 (segment (start 175.649 117.889686) (end 192.779686 100.759) (width 0.2) (layer "F.Cu") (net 1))
 (segment (start 190.388314 123.361) (end 180.1 123.361) (width 0.2) (layer "F.Cu") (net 1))
 (segment (start 189.89947 104.311) (end 179.886184 104.311) (width 0.2) (layer "F.Cu") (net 1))
 (segment (start 179.72925 86.039) (end 180.83025 84.938) (width 0.2) (layer "F.Cu") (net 1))
 (segment (start 180.1 131.75) (end 180.1 123.361) (width 0.2) (layer "F.Cu") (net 1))
 (segment (start 175.649 119.123816) (end 175.649 117.889686) (width 0.2) (layer "F.Cu") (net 1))
 (segment (start 174.57 91.19825) (end 180.83025 84.938) (width 0.2) (layer "F.Cu") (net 1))
 (segment (start 192.779686 100.759) (end 195.32747 100.759) (width 0.2) (layer "F.Cu") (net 1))
 (segment (start 194.699 119.050314) (end 190.454657 123.294657) (width 0.2) (layer "F.Cu") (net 1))
 (segment (start 175.649 95.23925) (end 180.83025 90.058) (width 0.2) (layer "F.Cu") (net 1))
 (segment (start 200.601314 134.96) (end 196.660314 138.901) (width 0.2) (layer "F.Cu") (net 1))
 (segment (start 195.499686 138.901) (end 190.454657 133.855971) (width 0.2) (layer "F.Cu") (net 1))
 (segment (start 179.886184 104.311) (end 175.649 100.073816) (width 0.2) (layer "F.Cu") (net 1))
 (segment (start 196.311836 101.46253) (end 200.894366 96.88) (width 0.2) (layer "F.Cu") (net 1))
 (segment (start 179.886184 123.361) (end 175.649 119.123816) (width 0.2) (layer "F.Cu") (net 1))
 (segment (start 183.4 96.88) (end 183.4 92.62775) (width 0.2) (layer "F.Cu") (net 1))
 (segment (start 196.660314 138.901) (end 195.499686 138.901) (width 0.2) (layer "F.Cu") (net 1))
 (segment (start 182.82825 88.556) (end 182.82825 85.186) (width 0.2) (layer "F.Cu") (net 16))
 (segment (start 182.82825 85.186) (end 180.83025 83.188) (width 0.2) (layer "F.Cu") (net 16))
 (segment (start 184.33025 90.058) (end 182.82825 88.556) (width 0.2) (layer "F.Cu") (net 16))
 (segment (start 183.22925 84.289) (end 183.22925 87.207) (width 0.2) (layer "F.Cu") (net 17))
 (segment (start 184.33025 83.188) (end 183.22925 84.289) (width 0.2) (layer "F.Cu") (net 17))
 (segment (start 183.22925 87.207) (end 184.33025 88.308) (width 0.2) (layer "F.Cu") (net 17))
 (segment (start 182.841314 99.42) (end 197.01125 85.250064) (width 0.2) (layer "F.Cu") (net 2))
 (segment (start 197.01125 85.250064) (end 197.01125 78.1475) (width 0.2) (layer "F.Cu") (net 2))
 (segment (start 177.05 99.42) (end 182.841314 99.42) (width 0.2) (layer "F.Cu") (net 2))
 (segment (start 199.36325 76.88187) (end 198.08888 75.6075) (width 0.2) (layer "F.Cu") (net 11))
 (segment (start 199.36325 96.15675) (end 199.36325 76.88187) (width 0.2) (layer "F.Cu") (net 11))
 (segment (start 198.08888 75.6075) (end 197.01125 75.6075) (width 0.2) (layer "F.Cu") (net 11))
 (segment (start 196.1 99.42) (end 199.36325 96.15675) (width 0.2) (layer "F.Cu") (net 11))
 (segment (start 200.228314 98.281) (end 203.030314 98.281) (width 0.2) (layer "F.Cu") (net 3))
 (segment (start 184.801 116.510314) (end 184.801 113.708314) (width 0.2) (layer "F.Cu") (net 3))
 (segment (start 203.851 97.460314) (end 203.851 79.07225) (width 0.2) (layer "F.Cu") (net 3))
 (segment (start 182.841314 118.47) (end 184.801 116.510314) (width 0.2) (layer "F.Cu") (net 3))
 (segment (start 177.05 118.47) (end 182.841314 118.47) (width 0.2) (layer "F.Cu") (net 3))
 (segment (start 203.030314 98.281) (end 203.851 97.460314) (width 0.2) (layer "F.Cu") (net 3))
 (segment (start 184.801 113.708314) (end 200.228314 98.281) (width 0.2) (layer "F.Cu") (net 3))
 (segment (start 203.851 79.07225) (end 197.84625 73.0675) (width 0.2) (layer "F.Cu") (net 3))
 (segment (start 206.28 78.71862) (end 198.08888 70.5275) (width 0.2) (layer "F.Cu") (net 12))
 (segment (start 198.08888 70.5275) (end 197.01125 70.5275) (width 0.2) (layer "F.Cu") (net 12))
 (segment (start 196.08 118.47) (end 196 118.39) (width 0.2) (layer "F.Cu") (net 12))
 (segment (start 196.1 118.47) (end 206.28 108.29) (width 0.2) (layer "F.Cu") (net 12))
 (segment (start 196.1 118.47) (end 196.08 118.47) (width 0.2) (layer "F.Cu") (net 12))
 (segment (start 206.28 108.29) (end 206.28 78.71862) (width 0.2) (layer "F.Cu") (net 12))
 (segment (start 177.05 137.59) (end 174.169 134.709) (width 0.2) (layer "F.Cu") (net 4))
 (segment (start 174.169 69.43212) (end 180.69362 62.9075) (width 0.2) (layer "F.Cu") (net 4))
 (segment (start 180.69362 62.9075) (end 181.77125 62.9075) (width 0.2) (layer "F.Cu") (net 4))
 (segment (start 174.169 134.709) (end 174.169 69.43212) (width 0.2) (layer "F.Cu") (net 4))
 (segment (start 206.681 77.043624) (end 198.687876 69.0505) (width 0.2) (layer "F.Cu") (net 5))
 (segment (start 196.08 137.5) (end 206.681 126.899) (width 0.2) (layer "F.Cu") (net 5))
 (segment (start 198.687876 69.0505) (end 185.37425 69.0505) (width 0.2) (layer "F.Cu") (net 5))
 (segment (start 185.37425 69.0505) (end 181.77125 65.4475) (width 0.2) (layer "F.Cu") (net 5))
 (segment (start 206.681 126.899) (end 206.681 77.043624) (width 0.2) (layer "F.Cu") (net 5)))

